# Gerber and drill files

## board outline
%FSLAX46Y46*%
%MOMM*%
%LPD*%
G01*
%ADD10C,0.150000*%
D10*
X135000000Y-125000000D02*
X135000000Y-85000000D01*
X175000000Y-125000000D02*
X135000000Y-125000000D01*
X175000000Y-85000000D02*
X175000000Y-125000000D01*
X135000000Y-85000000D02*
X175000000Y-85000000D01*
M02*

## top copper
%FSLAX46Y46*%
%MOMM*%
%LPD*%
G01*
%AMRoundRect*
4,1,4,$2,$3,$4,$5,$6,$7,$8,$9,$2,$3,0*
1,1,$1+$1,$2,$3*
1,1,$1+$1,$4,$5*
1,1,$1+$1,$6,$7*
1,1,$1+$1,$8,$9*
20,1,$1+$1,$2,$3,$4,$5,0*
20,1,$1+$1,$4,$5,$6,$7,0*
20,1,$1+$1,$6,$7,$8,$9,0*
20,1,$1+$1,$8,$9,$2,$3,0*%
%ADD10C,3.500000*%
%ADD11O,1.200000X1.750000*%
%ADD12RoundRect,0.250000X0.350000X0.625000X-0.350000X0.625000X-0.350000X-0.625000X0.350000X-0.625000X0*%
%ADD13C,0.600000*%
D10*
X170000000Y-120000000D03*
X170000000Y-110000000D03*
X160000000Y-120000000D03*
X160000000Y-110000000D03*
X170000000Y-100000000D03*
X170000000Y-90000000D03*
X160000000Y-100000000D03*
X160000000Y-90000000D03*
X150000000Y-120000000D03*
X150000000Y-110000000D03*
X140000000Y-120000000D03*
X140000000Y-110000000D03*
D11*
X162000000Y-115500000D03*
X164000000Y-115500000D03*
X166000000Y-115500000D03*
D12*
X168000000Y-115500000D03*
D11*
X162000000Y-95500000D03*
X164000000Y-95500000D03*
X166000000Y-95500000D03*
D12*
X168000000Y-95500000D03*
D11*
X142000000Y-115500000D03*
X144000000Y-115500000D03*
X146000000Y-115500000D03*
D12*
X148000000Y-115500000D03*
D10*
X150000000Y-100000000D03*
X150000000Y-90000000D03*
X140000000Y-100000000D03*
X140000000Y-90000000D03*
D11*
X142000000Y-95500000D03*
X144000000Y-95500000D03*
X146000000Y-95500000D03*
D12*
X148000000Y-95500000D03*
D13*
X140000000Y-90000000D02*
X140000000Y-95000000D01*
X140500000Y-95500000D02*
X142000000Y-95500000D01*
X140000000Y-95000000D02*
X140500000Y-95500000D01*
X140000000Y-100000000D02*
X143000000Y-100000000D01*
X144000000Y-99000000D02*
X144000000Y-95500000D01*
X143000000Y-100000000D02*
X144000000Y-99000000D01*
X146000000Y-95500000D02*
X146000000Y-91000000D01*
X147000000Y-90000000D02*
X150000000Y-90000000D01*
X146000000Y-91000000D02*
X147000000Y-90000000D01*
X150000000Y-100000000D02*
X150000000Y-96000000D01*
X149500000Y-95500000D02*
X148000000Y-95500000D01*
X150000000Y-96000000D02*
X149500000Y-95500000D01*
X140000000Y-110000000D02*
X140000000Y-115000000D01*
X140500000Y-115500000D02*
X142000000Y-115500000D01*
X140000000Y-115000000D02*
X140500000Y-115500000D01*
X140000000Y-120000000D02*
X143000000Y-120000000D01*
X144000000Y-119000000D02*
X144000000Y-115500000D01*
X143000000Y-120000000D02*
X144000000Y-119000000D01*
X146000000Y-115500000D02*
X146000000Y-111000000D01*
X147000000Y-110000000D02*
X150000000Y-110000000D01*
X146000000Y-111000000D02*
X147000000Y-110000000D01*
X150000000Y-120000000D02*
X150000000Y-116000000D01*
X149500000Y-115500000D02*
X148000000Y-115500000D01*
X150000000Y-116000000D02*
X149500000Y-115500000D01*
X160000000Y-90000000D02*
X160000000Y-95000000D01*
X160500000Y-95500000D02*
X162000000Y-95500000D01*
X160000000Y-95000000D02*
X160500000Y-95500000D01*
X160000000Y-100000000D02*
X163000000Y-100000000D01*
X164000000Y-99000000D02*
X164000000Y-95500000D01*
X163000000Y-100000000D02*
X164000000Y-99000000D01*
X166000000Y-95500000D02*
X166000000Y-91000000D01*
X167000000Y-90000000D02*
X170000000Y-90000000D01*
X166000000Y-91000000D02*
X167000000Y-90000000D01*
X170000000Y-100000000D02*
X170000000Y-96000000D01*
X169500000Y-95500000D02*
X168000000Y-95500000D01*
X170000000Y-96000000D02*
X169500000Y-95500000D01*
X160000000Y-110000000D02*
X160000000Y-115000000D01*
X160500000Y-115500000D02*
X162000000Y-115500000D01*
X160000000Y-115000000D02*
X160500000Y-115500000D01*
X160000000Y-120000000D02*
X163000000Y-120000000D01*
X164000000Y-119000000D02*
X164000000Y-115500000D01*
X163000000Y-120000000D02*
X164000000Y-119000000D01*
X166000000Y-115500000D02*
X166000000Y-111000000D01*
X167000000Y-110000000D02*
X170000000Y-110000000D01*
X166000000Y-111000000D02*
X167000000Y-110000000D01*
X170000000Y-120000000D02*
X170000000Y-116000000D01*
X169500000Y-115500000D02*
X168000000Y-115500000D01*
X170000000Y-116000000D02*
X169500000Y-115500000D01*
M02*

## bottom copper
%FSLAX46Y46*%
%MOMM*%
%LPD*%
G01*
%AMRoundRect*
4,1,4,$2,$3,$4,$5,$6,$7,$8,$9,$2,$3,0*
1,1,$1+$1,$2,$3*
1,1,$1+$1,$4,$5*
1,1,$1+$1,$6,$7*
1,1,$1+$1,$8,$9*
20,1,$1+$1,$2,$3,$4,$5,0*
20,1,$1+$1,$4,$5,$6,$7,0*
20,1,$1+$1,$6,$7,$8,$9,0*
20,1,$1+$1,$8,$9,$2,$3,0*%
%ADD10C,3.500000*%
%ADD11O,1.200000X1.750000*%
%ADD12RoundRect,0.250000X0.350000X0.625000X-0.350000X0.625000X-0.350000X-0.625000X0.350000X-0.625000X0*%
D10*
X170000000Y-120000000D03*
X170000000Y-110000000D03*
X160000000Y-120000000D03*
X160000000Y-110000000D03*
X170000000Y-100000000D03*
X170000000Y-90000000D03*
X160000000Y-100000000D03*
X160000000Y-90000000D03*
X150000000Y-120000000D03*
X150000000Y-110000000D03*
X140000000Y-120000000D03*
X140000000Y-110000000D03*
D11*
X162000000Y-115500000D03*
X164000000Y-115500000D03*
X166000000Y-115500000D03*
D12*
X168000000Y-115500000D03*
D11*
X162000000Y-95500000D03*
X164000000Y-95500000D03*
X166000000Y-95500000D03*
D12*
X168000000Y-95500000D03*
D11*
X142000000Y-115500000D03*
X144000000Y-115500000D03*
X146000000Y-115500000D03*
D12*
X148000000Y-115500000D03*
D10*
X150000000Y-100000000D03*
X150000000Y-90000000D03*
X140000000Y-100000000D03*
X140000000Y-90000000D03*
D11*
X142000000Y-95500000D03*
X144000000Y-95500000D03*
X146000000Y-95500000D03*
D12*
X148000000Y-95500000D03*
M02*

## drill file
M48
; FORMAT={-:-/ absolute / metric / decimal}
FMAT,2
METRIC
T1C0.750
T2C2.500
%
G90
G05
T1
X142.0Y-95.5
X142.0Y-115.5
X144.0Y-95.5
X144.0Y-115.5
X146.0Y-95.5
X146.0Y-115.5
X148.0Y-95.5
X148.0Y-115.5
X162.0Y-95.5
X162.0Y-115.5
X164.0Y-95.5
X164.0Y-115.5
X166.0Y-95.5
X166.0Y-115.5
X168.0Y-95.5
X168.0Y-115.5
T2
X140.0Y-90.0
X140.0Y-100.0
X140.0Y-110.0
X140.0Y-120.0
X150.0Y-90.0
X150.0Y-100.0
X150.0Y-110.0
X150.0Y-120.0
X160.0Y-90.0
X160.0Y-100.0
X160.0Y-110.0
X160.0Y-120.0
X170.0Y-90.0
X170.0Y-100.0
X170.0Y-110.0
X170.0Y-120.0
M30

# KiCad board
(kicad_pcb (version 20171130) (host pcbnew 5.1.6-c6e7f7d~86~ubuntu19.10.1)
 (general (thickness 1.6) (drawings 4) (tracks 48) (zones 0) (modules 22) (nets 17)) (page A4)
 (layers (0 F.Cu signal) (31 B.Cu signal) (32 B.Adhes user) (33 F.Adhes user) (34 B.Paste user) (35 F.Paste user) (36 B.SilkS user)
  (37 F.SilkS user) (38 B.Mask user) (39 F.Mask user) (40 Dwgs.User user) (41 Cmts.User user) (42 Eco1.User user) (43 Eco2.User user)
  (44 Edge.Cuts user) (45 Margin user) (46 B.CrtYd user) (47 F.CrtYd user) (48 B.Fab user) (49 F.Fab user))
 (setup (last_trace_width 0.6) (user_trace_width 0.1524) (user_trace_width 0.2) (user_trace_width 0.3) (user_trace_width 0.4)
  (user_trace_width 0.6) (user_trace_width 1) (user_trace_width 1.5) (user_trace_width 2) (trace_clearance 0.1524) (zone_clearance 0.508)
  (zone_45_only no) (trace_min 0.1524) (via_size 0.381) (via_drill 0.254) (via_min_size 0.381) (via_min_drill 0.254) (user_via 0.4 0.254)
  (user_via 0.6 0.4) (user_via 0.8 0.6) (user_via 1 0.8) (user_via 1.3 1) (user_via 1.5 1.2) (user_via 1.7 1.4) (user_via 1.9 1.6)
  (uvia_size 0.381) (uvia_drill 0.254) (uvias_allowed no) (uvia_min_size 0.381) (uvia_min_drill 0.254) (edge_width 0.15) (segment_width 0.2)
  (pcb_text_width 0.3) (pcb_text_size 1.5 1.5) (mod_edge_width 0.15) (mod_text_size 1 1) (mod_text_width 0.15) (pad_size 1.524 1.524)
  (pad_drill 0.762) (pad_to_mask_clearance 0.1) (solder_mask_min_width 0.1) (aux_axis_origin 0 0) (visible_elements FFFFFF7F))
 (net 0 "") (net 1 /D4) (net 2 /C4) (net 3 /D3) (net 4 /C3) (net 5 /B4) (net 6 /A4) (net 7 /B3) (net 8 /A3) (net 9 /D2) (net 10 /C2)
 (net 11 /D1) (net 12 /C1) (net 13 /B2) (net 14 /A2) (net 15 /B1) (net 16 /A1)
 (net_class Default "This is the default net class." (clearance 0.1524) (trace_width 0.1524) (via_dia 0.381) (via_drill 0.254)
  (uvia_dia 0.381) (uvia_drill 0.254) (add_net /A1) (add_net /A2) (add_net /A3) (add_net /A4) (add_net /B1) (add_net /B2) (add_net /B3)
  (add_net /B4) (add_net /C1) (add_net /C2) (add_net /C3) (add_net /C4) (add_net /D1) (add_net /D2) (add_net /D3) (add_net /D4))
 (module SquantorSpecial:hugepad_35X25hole (layer F.Cu) (at 170 120)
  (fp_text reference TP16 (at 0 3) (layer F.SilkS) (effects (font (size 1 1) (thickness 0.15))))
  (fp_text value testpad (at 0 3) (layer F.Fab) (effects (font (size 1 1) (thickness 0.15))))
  (pad 1 thru_hole circle (at 0 0) (size 3.5 3.5) (drill 2.5) (layers *.Cu *.Mask) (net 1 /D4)))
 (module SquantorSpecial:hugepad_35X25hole (layer F.Cu) (at 170 110)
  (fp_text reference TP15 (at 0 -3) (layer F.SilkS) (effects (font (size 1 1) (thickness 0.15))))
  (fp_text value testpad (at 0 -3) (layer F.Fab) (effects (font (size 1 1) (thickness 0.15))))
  (pad 1 thru_hole circle (at 0 0) (size 3.5 3.5) (drill 2.5) (layers *.Cu *.Mask) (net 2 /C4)))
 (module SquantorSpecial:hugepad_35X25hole (layer F.Cu) (at 160 120)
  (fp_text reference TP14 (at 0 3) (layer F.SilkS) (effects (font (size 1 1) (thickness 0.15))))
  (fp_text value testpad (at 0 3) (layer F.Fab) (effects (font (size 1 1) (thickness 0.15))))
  (pad 1 thru_hole circle (at 0 0) (size 3.5 3.5) (drill 2.5) (layers *.Cu *.Mask) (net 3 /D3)))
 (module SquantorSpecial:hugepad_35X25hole (layer F.Cu) (at 160 110)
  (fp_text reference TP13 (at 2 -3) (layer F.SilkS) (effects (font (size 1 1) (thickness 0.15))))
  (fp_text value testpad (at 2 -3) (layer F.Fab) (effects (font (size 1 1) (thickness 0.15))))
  (pad 1 thru_hole circle (at 0 0) (size 3.5 3.5) (drill 2.5) (layers *.Cu *.Mask) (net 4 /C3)))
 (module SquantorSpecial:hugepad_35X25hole (layer F.Cu) (at 170 100)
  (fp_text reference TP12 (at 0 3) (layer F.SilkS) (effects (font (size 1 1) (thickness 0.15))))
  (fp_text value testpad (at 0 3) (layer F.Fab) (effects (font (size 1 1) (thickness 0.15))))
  (pad 1 thru_hole circle (at 0 0) (size 3.5 3.5) (drill 2.5) (layers *.Cu *.Mask) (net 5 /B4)))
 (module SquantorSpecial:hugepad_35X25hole (layer F.Cu) (at 170 90)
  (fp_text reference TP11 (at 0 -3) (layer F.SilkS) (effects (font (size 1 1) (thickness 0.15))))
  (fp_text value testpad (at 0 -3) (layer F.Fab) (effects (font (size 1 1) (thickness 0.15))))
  (pad 1 thru_hole circle (at 0 0) (size 3.5 3.5) (drill 2.5) (layers *.Cu *.Mask) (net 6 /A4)))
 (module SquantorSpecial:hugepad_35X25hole (layer F.Cu) (at 160 100)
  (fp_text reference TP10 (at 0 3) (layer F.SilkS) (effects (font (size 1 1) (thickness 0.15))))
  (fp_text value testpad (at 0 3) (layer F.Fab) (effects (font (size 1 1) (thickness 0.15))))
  (pad 1 thru_hole circle (at 0 0) (size 3.5 3.5) (drill 2.5) (layers *.Cu *.Mask) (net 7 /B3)))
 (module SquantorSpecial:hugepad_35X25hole (layer F.Cu) (at 160 90)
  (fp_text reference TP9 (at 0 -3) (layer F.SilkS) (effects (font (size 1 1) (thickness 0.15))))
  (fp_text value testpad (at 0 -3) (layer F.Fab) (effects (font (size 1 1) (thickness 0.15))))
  (pad 1 thru_hole circle (at 0 0) (size 3.5 3.5) (drill 2.5) (layers *.Cu *.Mask) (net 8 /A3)))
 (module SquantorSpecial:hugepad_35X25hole (layer F.Cu) (at 150 120)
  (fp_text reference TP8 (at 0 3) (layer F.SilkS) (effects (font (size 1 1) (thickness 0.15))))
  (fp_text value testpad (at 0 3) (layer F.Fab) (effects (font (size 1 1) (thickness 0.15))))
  (pad 1 thru_hole circle (at 0 0) (size 3.5 3.5) (drill 2.5) (layers *.Cu *.Mask) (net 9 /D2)))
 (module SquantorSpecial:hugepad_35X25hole (layer F.Cu) (at 150 110)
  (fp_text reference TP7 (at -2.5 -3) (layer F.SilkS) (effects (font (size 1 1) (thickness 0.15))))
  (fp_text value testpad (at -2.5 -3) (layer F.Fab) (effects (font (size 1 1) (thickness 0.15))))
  (pad 1 thru_hole circle (at 0 0) (size 3.5 3.5) (drill 2.5) (layers *.Cu *.Mask) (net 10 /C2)))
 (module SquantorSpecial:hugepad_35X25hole (layer F.Cu) (at 140 120)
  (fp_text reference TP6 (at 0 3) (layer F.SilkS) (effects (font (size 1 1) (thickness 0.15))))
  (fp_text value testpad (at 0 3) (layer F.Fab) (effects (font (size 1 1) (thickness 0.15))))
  (pad 1 thru_hole circle (at 0 0) (size 3.5 3.5) (drill 2.5) (layers *.Cu *.Mask) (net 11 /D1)))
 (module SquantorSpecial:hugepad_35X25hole (layer F.Cu) (at 140 110)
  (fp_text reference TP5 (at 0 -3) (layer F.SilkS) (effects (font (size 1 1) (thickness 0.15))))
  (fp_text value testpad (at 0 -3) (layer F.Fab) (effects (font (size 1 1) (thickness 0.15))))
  (pad 1 thru_hole circle (at 0 0) (size 3.5 3.5) (drill 2.5) (layers *.Cu *.Mask) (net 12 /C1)))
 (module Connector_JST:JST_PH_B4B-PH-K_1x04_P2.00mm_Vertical (layer F.Cu) (at 168 115.5 180)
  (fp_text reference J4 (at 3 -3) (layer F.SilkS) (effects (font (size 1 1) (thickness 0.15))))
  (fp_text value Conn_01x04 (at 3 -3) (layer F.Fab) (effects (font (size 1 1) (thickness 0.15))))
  (pad 4 thru_hole oval (at 6 0 180) (size 1.2 1.75) (drill 0.75) (layers *.Cu *.Mask) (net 4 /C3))
  (pad 3 thru_hole oval (at 4 0 180) (size 1.2 1.75) (drill 0.75) (layers *.Cu *.Mask) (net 3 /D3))
  (pad 2 thru_hole oval (at 2 0 180) (size 1.2 1.75) (drill 0.75) (layers *.Cu *.Mask) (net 2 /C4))
  (pad 1 thru_hole roundrect (at 0 0 180) (size 1.2 1.75) (drill 0.75) (layers *.Cu *.Mask) (roundrect_rratio 0.208333) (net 1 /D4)))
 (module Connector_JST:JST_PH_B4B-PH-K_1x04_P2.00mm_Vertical (layer F.Cu) (at 168 95.5 180)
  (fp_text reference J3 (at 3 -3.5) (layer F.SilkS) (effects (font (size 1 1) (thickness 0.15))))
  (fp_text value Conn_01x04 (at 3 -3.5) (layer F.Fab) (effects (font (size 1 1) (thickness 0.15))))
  (pad 4 thru_hole oval (at 6 0 180) (size 1.2 1.75) (drill 0.75) (layers *.Cu *.Mask) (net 8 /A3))
  (pad 3 thru_hole oval (at 4 0 180) (size 1.2 1.75) (drill 0.75) (layers *.Cu *.Mask) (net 7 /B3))
  (pad 2 thru_hole oval (at 2 0 180) (size 1.2 1.75) (drill 0.75) (layers *.Cu *.Mask) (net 6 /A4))
  (pad 1 thru_hole roundrect (at 0 0 180) (size 1.2 1.75) (drill 0.75) (layers *.Cu *.Mask) (roundrect_rratio 0.208333) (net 5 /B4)))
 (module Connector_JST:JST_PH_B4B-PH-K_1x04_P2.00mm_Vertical (layer F.Cu) (at 148 115.5 180)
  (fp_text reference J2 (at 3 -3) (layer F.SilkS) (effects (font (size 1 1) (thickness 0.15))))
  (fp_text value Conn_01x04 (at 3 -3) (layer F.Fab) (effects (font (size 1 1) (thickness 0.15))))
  (pad 4 thru_hole oval (at 6 0 180) (size 1.2 1.75) (drill 0.75) (layers *.Cu *.Mask) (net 12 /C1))
  (pad 3 thru_hole oval (at 4 0 180) (size 1.2 1.75) (drill 0.75) (layers *.Cu *.Mask) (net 11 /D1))
  (pad 2 thru_hole oval (at 2 0 180) (size 1.2 1.75) (drill 0.75) (layers *.Cu *.Mask) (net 10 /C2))
  (pad 1 thru_hole roundrect (at 0 0 180) (size 1.2 1.75) (drill 0.75) (layers *.Cu *.Mask) (roundrect_rratio 0.208333) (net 9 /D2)))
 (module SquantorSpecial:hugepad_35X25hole (layer F.Cu) (at 150 100)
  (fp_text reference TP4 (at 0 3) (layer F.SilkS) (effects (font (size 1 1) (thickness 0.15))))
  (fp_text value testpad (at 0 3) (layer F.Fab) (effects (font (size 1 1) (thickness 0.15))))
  (pad 1 thru_hole circle (at 0 0) (size 3.5 3.5) (drill 2.5) (layers *.Cu *.Mask) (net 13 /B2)))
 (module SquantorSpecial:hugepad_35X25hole (layer F.Cu) (at 150 90)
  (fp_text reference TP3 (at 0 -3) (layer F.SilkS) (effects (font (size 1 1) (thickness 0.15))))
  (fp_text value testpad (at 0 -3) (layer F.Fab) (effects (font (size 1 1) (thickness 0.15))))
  (pad 1 thru_hole circle (at 0 0) (size 3.5 3.5) (drill 2.5) (layers *.Cu *.Mask) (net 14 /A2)))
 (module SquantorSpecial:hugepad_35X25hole (layer F.Cu) (at 140 100)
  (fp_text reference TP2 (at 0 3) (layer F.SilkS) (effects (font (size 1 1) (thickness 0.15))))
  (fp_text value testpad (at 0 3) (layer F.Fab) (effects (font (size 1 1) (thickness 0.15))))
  (pad 1 thru_hole circle (at 0 0) (size 3.5 3.5) (drill 2.5) (layers *.Cu *.Mask) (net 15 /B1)))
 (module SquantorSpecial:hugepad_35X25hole (layer F.Cu) (at 140 90)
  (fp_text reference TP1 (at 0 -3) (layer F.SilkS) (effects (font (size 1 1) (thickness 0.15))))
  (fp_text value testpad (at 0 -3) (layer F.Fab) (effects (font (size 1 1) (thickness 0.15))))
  (pad 1 thru_hole circle (at 0 0) (size 3.5 3.5) (drill 2.5) (layers *.Cu *.Mask) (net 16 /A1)))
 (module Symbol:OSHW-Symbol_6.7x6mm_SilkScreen (layer F.Cu) (at 155 103)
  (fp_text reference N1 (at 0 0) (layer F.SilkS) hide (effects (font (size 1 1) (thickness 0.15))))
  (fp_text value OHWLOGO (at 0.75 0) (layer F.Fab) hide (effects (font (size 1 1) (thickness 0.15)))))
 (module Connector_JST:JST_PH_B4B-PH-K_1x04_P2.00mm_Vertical (layer F.Cu) (at 148 95.5 180)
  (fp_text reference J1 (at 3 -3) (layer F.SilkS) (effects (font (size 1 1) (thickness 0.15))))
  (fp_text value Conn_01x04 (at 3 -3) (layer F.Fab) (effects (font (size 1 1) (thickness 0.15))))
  (pad 4 thru_hole oval (at 6 0 180) (size 1.2 1.75) (drill 0.75) (layers *.Cu *.Mask) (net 16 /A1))
  (pad 3 thru_hole oval (at 4 0 180) (size 1.2 1.75) (drill 0.75) (layers *.Cu *.Mask) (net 15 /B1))
  (pad 2 thru_hole oval (at 2 0 180) (size 1.2 1.75) (drill 0.75) (layers *.Cu *.Mask) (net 14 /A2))
  (pad 1 thru_hole roundrect (at 0 0 180) (size 1.2 1.75) (drill 0.75) (layers *.Cu *.Mask) (roundrect_rratio 0.208333) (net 13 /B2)))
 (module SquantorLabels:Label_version (layer F.Cu) (at 156 107)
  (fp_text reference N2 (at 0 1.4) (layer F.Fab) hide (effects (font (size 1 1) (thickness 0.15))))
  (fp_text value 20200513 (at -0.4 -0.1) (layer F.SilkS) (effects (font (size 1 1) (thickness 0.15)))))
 (gr_line (start 135 125) (end 135 85) (layer Edge.Cuts) (width 0.15))
 (gr_line (start 175 125) (end 135 125) (layer Edge.Cuts) (width 0.15))
 (gr_line (start 175 85) (end 175 125) (layer Edge.Cuts) (width 0.15))
 (gr_line (start 135 85) (end 175 85) (layer Edge.Cuts) (width 0.15))
 (segment (start 140 90) (end 140 95) (width 0.6) (layer F.Cu) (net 16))
 (segment (start 140.5 95.5) (end 142 95.5) (width 0.6) (layer F.Cu) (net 16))
 (segment (start 140 95) (end 140.5 95.5) (width 0.6) (layer F.Cu) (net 16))
 (segment (start 140 100) (end 143 100) (width 0.6) (layer F.Cu) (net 15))
 (segment (start 144 99) (end 144 95.5) (width 0.6) (layer F.Cu) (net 15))
 (segment (start 143 100) (end 144 99) (width 0.6) (layer F.Cu) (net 15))
 (segment (start 146 95.5) (end 146 91) (width 0.6) (layer F.Cu) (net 14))
 (segment (start 147 90) (end 150 90) (width 0.6) (layer F.Cu) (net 14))
 (segment (start 146 91) (end 147 90) (width 0.6) (layer F.Cu) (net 14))
 (segment (start 150 100) (end 150 96) (width 0.6) (layer F.Cu) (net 13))
 (segment (start 149.5 95.5) (end 148 95.5) (width 0.6) (layer F.Cu) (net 13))
 (segment (start 150 96) (end 149.5 95.5) (width 0.6) (layer F.Cu) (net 13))
 (segment (start 140 110) (end 140 115) (width 0.6) (layer F.Cu) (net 12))
 (segment (start 140.5 115.5) (end 142 115.5) (width 0.6) (layer F.Cu) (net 12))
 (segment (start 140 115) (end 140.5 115.5) (width 0.6) (layer F.Cu) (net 12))
 (segment (start 140 120) (end 143 120) (width 0.6) (layer F.Cu) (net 11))
 (segment (start 144 119) (end 144 115.5) (width 0.6) (layer F.Cu) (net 11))
 (segment (start 143 120) (end 144 119) (width 0.6) (layer F.Cu) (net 11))
 (segment (start 146 115.5) (end 146 111) (width 0.6) (layer F.Cu) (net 10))
 (segment (start 147 110) (end 150 110) (width 0.6) (layer F.Cu) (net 10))
 (segment (start 146 111) (end 147 110) (width 0.6) (layer F.Cu) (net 10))
 (segment (start 150 120) (end 150 116) (width 0.6) (layer F.Cu) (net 9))
 (segment (start 149.5 115.5) (end 148 115.5) (width 0.6) (layer F.Cu) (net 9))
 (segment (start 150 116) (end 149.5 115.5) (width 0.6) (layer F.Cu) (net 9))
 (segment (start 160 90) (end 160 95) (width 0.6) (layer F.Cu) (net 8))
 (segment (start 160.5 95.5) (end 162 95.5) (width 0.6) (layer F.Cu) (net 8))
 (segment (start 160 95) (end 160.5 95.5) (width 0.6) (layer F.Cu) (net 8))
 (segment (start 160 100) (end 163 100) (width 0.6) (layer F.Cu) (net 7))
 (segment (start 164 99) (end 164 95.5) (width 0.6) (layer F.Cu) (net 7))
 (segment (start 163 100) (end 164 99) (width 0.6) (layer F.Cu) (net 7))
 (segment (start 166 95.5) (end 166 91) (width 0.6) (layer F.Cu) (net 6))
 (segment (start 167 90) (end 170 90) (width 0.6) (layer F.Cu) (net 6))
 (segment (start 166 91) (end 167 90) (width 0.6) (layer F.Cu) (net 6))
 (segment (start 170 100) (end 170 96) (width 0.6) (layer F.Cu) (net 5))
 (segment (start 169.5 95.5) (end 168 95.5) (width 0.6) (layer F.Cu) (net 5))
 (segment (start 170 96) (end 169.5 95.5) (width 0.6) (layer F.Cu) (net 5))
 (segment (start 160 110) (end 160 115) (width 0.6) (layer F.Cu) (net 4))
 (segment (start 160.5 115.5) (end 162 115.5) (width 0.6) (layer F.Cu) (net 4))
 (segment (start 160 115) (end 160.5 115.5) (width 0.6) (layer F.Cu) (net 4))
 (segment (start 160 120) (end 163 120) (width 0.6) (layer F.Cu) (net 3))
 (segment (start 164 119) (end 164 115.5) (width 0.6) (layer F.Cu) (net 3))
 (segment (start 163 120) (end 164 119) (width 0.6) (layer F.Cu) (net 3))
 (segment (start 166 115.5) (end 166 111) (width 0.6) (layer F.Cu) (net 2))
 (segment (start 167 110) (end 170 110) (width 0.6) (layer F.Cu) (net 2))
 (segment (start 166 111) (end 167 110) (width 0.6) (layer F.Cu) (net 2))
 (segment (start 170 120) (end 170 116) (width 0.6) (layer F.Cu) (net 1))
 (segment (start 169.5 115.5) (end 168 115.5) (width 0.6) (layer F.Cu) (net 1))
 (segment (start 170 116) (end 169.5 115.5) (width 0.6) (layer F.Cu) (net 1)))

